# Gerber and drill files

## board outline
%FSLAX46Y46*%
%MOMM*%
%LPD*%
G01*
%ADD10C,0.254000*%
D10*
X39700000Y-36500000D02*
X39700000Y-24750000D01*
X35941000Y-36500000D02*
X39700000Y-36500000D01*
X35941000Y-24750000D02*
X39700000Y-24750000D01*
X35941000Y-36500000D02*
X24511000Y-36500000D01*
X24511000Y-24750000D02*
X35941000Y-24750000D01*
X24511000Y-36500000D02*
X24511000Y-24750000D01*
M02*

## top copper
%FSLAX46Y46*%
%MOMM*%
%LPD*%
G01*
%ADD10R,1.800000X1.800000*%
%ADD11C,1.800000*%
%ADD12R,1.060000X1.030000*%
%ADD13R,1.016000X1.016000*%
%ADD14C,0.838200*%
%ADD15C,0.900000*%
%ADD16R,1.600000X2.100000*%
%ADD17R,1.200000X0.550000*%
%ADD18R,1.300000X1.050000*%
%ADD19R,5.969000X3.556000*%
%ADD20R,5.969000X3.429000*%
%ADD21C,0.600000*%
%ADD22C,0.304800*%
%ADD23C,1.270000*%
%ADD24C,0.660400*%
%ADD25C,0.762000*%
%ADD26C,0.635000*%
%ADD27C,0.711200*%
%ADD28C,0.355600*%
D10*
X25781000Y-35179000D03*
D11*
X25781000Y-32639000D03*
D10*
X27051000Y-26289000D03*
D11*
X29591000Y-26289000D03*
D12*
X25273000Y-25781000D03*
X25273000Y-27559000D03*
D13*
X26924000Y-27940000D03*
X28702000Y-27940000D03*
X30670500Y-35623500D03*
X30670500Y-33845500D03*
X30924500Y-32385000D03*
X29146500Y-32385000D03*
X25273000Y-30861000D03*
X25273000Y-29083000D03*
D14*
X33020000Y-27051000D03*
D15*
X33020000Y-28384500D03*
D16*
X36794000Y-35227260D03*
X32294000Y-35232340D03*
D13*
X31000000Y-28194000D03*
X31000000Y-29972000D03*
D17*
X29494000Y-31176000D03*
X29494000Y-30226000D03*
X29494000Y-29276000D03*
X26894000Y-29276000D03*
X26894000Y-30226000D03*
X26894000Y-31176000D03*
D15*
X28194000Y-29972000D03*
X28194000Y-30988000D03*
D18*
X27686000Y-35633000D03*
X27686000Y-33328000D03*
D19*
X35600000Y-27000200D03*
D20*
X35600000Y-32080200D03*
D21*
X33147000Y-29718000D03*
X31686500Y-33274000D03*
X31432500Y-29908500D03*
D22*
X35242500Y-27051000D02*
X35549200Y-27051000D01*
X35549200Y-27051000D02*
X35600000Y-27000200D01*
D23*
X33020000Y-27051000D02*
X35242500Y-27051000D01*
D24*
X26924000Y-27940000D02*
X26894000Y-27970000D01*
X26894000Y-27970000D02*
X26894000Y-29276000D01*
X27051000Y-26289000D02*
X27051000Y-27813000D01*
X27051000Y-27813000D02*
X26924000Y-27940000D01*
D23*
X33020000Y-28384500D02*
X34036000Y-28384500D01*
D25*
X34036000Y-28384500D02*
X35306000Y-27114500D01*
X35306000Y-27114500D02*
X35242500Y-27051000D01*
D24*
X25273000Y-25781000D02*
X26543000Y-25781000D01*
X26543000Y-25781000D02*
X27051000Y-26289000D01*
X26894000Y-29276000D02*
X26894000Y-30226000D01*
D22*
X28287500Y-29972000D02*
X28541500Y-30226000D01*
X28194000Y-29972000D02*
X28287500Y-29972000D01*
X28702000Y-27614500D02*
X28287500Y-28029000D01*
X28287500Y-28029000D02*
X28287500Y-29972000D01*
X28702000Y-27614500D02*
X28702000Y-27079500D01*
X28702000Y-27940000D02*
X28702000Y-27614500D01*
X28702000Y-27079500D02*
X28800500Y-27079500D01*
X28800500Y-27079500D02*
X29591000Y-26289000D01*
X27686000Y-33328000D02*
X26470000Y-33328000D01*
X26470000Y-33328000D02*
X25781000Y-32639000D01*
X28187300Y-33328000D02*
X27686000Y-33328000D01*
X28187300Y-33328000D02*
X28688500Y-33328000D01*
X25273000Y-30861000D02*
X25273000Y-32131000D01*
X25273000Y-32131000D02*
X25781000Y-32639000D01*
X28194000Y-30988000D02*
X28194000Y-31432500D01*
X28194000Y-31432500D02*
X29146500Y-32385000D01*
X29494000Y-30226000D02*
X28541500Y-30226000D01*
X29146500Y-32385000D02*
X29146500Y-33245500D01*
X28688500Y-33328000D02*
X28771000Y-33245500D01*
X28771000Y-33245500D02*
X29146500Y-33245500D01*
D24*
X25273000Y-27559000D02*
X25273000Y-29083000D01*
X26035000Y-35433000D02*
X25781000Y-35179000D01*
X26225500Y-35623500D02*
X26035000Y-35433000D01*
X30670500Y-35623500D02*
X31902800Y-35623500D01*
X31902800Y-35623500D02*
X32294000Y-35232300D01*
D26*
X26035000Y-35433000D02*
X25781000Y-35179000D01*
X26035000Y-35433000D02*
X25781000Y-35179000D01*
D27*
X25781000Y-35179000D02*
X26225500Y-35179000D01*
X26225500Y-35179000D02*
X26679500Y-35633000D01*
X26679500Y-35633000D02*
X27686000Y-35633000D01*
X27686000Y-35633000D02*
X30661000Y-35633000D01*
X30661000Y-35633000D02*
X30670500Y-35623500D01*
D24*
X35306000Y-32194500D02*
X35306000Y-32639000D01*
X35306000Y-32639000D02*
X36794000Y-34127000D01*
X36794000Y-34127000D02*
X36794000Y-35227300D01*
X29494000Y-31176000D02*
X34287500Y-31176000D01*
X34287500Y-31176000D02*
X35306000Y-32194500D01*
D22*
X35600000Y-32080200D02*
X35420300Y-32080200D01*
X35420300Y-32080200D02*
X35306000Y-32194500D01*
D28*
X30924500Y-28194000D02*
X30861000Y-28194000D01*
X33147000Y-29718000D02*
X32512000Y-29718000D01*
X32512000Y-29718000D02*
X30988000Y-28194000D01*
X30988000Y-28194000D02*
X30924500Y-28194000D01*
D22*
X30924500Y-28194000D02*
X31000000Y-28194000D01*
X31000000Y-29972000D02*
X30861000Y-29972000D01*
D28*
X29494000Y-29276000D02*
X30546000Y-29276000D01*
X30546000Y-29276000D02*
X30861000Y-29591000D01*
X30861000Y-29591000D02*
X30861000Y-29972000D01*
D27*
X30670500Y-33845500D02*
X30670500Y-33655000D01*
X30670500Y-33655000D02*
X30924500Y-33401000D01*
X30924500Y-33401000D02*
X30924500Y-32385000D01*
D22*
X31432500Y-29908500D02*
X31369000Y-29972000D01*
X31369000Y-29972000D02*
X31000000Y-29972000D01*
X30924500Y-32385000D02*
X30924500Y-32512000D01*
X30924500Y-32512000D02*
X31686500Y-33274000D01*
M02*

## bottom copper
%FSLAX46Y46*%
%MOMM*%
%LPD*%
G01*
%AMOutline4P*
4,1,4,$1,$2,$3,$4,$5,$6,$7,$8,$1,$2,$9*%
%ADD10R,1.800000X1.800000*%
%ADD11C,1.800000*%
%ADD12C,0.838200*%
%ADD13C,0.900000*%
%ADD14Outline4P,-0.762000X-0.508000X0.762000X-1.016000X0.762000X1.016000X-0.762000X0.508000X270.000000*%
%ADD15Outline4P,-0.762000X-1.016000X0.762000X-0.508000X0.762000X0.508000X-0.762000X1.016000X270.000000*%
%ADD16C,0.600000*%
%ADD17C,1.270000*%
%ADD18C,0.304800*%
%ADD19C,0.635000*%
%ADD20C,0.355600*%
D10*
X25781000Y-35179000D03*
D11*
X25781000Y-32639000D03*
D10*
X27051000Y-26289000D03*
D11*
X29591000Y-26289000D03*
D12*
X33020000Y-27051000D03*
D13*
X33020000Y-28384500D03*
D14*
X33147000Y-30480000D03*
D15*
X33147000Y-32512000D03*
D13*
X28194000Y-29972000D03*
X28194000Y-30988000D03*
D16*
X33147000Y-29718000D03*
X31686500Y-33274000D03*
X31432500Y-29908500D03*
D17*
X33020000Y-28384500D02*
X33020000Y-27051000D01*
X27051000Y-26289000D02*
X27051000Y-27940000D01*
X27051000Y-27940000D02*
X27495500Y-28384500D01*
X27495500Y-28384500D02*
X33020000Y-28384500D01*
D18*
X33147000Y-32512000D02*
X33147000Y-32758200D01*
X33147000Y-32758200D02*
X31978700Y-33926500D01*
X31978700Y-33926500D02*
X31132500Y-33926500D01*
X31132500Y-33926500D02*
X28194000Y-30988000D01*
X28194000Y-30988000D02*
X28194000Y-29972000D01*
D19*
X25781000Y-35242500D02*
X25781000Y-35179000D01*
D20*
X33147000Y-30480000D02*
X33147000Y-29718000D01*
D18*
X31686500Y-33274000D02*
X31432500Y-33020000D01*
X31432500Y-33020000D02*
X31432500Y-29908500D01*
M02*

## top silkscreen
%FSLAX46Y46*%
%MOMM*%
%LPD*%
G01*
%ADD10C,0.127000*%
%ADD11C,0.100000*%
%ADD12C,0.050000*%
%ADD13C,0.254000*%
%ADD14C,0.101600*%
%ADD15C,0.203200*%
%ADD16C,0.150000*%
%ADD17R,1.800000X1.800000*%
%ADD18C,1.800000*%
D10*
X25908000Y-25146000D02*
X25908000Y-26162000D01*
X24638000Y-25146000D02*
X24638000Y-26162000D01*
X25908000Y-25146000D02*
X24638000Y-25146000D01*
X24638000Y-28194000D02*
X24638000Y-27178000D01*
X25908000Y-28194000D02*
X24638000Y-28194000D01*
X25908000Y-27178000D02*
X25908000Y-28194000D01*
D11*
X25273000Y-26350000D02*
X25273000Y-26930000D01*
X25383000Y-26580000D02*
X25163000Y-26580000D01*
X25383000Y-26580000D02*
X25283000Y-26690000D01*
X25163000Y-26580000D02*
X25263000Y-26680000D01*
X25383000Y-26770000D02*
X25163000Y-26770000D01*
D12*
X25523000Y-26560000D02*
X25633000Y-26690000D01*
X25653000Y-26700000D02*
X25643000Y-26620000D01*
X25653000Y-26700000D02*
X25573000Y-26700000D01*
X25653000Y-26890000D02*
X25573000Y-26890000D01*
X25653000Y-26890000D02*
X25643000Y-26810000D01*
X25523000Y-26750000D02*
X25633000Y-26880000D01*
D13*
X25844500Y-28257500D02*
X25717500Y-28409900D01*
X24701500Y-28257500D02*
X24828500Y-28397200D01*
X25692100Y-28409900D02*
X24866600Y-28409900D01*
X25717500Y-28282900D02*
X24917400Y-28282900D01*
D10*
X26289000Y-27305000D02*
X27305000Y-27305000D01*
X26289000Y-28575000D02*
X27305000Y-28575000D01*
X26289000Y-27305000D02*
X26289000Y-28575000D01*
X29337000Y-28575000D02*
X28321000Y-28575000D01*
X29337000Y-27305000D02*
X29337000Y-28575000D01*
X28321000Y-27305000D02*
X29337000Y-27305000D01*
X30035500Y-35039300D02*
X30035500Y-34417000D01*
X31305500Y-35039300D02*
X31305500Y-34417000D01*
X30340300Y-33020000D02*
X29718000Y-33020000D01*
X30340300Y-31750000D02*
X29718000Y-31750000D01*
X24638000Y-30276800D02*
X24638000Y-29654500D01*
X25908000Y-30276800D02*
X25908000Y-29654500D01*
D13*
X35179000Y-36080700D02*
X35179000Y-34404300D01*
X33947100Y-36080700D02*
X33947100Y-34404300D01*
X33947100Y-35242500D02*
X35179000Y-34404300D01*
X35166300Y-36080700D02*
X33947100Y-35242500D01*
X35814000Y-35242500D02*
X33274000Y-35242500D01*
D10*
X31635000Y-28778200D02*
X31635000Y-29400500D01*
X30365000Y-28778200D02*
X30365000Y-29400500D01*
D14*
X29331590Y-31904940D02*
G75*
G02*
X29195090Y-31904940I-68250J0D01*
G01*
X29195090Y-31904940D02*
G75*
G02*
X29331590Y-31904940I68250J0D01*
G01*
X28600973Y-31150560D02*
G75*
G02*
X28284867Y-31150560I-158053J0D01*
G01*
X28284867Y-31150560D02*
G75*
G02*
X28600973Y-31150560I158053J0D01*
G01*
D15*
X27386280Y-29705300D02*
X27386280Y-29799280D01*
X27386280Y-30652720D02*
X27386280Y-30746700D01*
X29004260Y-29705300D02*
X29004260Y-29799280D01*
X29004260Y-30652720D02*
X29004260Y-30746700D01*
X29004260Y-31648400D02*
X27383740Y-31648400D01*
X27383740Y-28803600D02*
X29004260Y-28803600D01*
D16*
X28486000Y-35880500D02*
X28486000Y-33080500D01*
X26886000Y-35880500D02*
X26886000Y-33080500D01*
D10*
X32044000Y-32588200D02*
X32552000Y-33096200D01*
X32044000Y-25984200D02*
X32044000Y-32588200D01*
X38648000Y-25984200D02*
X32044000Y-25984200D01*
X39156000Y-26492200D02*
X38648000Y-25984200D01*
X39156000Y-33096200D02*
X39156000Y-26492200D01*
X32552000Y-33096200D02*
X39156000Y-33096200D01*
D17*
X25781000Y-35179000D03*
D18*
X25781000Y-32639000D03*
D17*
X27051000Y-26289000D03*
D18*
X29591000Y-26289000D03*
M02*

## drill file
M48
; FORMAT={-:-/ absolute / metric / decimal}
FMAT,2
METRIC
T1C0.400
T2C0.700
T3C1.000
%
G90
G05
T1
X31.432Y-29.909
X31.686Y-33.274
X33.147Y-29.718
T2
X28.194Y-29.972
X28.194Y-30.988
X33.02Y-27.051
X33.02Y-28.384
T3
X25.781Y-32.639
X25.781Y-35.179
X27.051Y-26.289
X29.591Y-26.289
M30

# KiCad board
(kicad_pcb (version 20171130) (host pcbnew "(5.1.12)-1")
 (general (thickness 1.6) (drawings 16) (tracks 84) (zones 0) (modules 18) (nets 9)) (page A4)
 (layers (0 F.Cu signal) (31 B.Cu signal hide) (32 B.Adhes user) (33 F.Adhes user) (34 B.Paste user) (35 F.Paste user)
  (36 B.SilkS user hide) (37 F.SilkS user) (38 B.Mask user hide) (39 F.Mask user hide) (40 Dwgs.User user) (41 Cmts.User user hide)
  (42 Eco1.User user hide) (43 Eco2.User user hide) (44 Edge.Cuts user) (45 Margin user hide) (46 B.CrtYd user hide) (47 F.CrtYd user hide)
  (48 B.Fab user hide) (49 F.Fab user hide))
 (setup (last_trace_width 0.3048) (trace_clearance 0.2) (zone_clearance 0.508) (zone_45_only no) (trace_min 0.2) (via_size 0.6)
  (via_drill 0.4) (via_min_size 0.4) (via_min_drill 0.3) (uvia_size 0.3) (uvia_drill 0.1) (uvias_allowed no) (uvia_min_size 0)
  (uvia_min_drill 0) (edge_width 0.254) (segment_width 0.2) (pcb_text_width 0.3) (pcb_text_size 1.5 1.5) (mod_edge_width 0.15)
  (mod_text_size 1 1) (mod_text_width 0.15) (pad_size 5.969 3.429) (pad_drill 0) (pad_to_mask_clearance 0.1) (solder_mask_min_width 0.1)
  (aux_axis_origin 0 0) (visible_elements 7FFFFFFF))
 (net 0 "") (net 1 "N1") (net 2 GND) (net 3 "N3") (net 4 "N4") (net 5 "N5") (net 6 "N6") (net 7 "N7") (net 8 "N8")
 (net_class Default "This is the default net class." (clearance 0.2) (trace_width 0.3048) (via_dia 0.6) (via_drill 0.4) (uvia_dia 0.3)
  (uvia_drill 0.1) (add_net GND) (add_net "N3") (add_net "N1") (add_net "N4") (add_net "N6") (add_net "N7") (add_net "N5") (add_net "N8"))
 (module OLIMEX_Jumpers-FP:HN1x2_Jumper (layer F.Cu) (at 25.781 33.909 90)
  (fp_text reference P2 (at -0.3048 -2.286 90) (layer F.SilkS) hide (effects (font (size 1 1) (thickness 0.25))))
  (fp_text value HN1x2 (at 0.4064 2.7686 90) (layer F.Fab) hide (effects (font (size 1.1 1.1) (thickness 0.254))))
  (pad 1 thru_hole rect (at -1.27 0 180) (size 1.8 1.8) (drill 1) (layers *.Cu *.Mask F.SilkS) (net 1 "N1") (solder_mask_margin 0.0508)
   (solder_paste_margin -0.0508))
  (pad 2 thru_hole circle (at 1.27 0 180) (size 1.8 1.8) (drill 1) (layers *.Cu *.Mask F.SilkS) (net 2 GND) (solder_mask_margin 0.0508)
   (solder_paste_margin -0.0508)))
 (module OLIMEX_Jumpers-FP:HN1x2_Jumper (layer F.Cu) (at 28.321 26.289)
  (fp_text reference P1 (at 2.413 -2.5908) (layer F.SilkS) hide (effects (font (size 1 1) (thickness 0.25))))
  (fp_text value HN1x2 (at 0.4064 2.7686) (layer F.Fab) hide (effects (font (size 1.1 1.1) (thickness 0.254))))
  (pad 1 thru_hole rect (at -1.27 0 90) (size 1.8 1.8) (drill 1) (layers *.Cu *.Mask F.SilkS) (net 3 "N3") (solder_mask_margin 0.0508)
   (solder_paste_margin -0.0508))
  (pad 2 thru_hole circle (at 1.27 0 90) (size 1.8 1.8) (drill 1) (layers *.Cu *.Mask F.SilkS) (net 2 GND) (solder_mask_margin 0.0508)
   (solder_paste_margin -0.0508)))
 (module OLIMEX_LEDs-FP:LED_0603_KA (layer F.Cu) (at 25.273 26.67 270)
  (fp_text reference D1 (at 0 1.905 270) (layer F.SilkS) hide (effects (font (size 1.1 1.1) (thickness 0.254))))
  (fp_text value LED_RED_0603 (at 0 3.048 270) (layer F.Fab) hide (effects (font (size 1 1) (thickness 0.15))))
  (fp_line (start -1.524 -0.635) (end -0.508 -0.635) (layer F.SilkS) (width 0.127))
  (fp_line (start -1.524 0.635) (end -0.508 0.635) (layer F.SilkS) (width 0.127))
  (fp_line (start -1.524 -0.635) (end -1.524 0.635) (layer F.SilkS) (width 0.127))
  (fp_line (start 1.524 0.635) (end 0.508 0.635) (layer F.SilkS) (width 0.127))
  (fp_line (start 1.524 -0.635) (end 1.524 0.635) (layer F.SilkS) (width 0.127))
  (fp_line (start 0.508 -0.635) (end 1.524 -0.635) (layer F.SilkS) (width 0.127))
  (fp_line (start -0.32 0) (end 0.26 0) (layer F.SilkS) (width 0.1))
  (fp_line (start -0.09 -0.11) (end -0.09 0.11) (layer F.SilkS) (width 0.1))
  (fp_line (start -0.09 -0.11) (end 0.02 -0.01) (layer F.SilkS) (width 0.1))
  (fp_line (start -0.09 0.11) (end 0.01 0.01) (layer F.SilkS) (width 0.1))
  (fp_line (start 0.1 -0.11) (end 0.1 0.11) (layer F.SilkS) (width 0.1))
  (fp_line (start -0.11 -0.25) (end 0.02 -0.36) (layer F.SilkS) (width 0.05))
  (fp_line (start 0.03 -0.38) (end -0.05 -0.37) (layer F.SilkS) (width 0.05))
  (fp_line (start 0.03 -0.38) (end 0.03 -0.3) (layer F.SilkS) (width 0.05))
  (fp_line (start 0.22 -0.38) (end 0.22 -0.3) (layer F.SilkS) (width 0.05))
  (fp_line (start 0.22 -0.38) (end 0.14 -0.37) (layer F.SilkS) (width 0.05))
  (fp_line (start 0.08 -0.25) (end 0.21 -0.36) (layer F.SilkS) (width 0.05))
  (fp_line (start 1.5875 -0.5715) (end 1.7399 -0.4445) (layer F.SilkS) (width 0.254))
  (fp_line (start 1.5875 0.5715) (end 1.7272 0.4445) (layer F.SilkS) (width 0.254))
  (fp_line (start 1.7399 -0.4191) (end 1.7399 0.4064) (layer F.SilkS) (width 0.254))
  (fp_line (start 1.6129 -0.4445) (end 1.6129 0.3556) (layer F.SilkS) (width 0.254))
  (pad 2 smd rect (at -0.889 0 270) (size 1.03 1.06) (layers F.Cu F.Paste F.Mask) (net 3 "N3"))
  (pad 1 smd rect (at 0.889 0 270) (size 1.03 1.06) (layers F.Cu F.Paste F.Mask) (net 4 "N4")))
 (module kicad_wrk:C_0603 (layer F.Cu) (at 27.813 27.94)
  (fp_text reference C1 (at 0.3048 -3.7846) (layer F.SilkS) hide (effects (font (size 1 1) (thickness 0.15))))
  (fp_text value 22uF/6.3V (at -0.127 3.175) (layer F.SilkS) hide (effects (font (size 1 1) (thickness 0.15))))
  (fp_line (start -1.524 -0.635) (end -0.508 -0.635) (layer F.SilkS) (width 0.127))
  (fp_line (start -1.524 0.635) (end -0.508 0.635) (layer F.SilkS) (width 0.127))
  (fp_line (start -1.524 -0.635) (end -1.524 0.635) (layer F.SilkS) (width 0.127))
  (fp_line (start 1.524 0.635) (end 0.508 0.635) (layer F.SilkS) (width 0.127))
  (fp_line (start 1.524 -0.635) (end 1.524 0.635) (layer F.SilkS) (width 0.127))
  (fp_line (start 0.508 -0.635) (end 1.524 -0.635) (layer F.SilkS) (width 0.127))
  (pad 1 smd rect (at -0.889 0) (size 1.016 1.016) (layers F.Cu F.Paste F.Mask) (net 3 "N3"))
  (pad 2 smd rect (at 0.889 0) (size 1.016 1.016) (layers F.Cu F.Paste F.Mask) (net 2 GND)))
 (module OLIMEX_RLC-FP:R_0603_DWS (layer F.Cu) (at 30.6705 34.7345 90)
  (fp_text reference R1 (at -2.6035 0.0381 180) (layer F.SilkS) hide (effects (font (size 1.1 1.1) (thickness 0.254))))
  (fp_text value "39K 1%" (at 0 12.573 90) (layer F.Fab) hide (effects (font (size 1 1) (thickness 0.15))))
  (fp_line (start -0.3048 -0.635) (end 0.3175 -0.635) (layer F.SilkS) (width 0.127))
  (fp_line (start -0.3048 0.635) (end 0.3175 0.635) (layer F.SilkS) (width 0.127))
  (pad 1 smd rect (at -0.889 0 90) (size 1.016 1.016) (layers F.Cu F.Paste F.Mask) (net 1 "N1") (solder_mask_margin 0.0508)
   (solder_paste_margin -0.0508) (clearance 0.0508))
  (pad 2 smd rect (at 0.889 0 90) (size 1.016 1.016) (layers F.Cu F.Paste F.Mask) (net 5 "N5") (solder_mask_margin 0.0508)
   (solder_paste_margin -0.0508) (clearance 0.0508)))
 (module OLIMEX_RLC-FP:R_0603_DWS (layer F.Cu) (at 30.0355 32.385 180)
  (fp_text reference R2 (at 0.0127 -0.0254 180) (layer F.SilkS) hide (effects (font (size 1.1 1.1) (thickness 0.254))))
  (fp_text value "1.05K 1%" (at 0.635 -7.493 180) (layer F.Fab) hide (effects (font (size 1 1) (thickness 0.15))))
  (fp_line (start -0.3048 -0.635) (end 0.3175 -0.635) (layer F.SilkS) (width 0.127))
  (fp_line (start -0.3048 0.635) (end 0.3175 0.635) (layer F.SilkS) (width 0.127))
  (pad 1 smd rect (at -0.889 0 180) (size 1.016 1.016) (layers F.Cu F.Paste F.Mask) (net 5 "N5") (solder_mask_margin 0.0508)
   (solder_paste_margin -0.0508) (clearance 0.0508))
  (pad 2 smd rect (at 0.889 0 180) (size 1.016 1.016) (layers F.Cu F.Paste F.Mask) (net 2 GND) (solder_mask_margin 0.0508)
   (solder_paste_margin -0.0508) (clearance 0.0508)))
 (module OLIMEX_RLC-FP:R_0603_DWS (layer F.Cu) (at 25.273 29.972 90)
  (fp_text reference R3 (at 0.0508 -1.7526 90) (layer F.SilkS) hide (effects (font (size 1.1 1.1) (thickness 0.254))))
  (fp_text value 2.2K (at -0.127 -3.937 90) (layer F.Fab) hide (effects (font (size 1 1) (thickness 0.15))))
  (fp_line (start -0.3048 -0.635) (end 0.3175 -0.635) (layer F.SilkS) (width 0.127))
  (fp_line (start -0.3048 0.635) (end 0.3175 0.635) (layer F.SilkS) (width 0.127))
  (pad 1 smd rect (at -0.889 0 90) (size 1.016 1.016) (layers F.Cu F.Paste F.Mask) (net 2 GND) (solder_mask_margin 0.0508)
   (solder_paste_margin -0.0508) (clearance 0.0508))
  (pad 2 smd rect (at 0.889 0 90) (size 1.016 1.016) (layers F.Cu F.Paste F.Mask) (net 4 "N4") (solder_mask_margin 0.0508)
   (solder_paste_margin -0.0508) (clearance 0.0508)))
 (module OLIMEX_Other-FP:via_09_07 (layer F.Cu) (at 33.02 27.051 180)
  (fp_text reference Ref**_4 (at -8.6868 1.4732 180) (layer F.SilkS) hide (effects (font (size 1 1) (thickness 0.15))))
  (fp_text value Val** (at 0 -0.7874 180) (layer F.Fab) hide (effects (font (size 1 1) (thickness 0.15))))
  (pad 0 thru_hole circle (at 0 0 180) (size 0.8382 0.8382) (drill 0.7) (layers *.Cu) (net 3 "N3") (zone_connect 2)))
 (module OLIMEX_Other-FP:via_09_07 (layer F.Cu) (at 33.02 28.321 180)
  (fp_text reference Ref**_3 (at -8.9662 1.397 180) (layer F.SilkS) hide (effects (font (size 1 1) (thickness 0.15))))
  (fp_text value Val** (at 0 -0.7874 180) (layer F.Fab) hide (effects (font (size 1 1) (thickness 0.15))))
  (pad 0 thru_hole circle (at 0 -0.0635 180) (size 0.9 0.9) (drill 0.7) (layers *.Cu) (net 3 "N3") (zone_connect 2)))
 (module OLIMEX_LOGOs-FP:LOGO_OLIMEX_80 (layer B.Cu) (at 35.8775 27.686 180)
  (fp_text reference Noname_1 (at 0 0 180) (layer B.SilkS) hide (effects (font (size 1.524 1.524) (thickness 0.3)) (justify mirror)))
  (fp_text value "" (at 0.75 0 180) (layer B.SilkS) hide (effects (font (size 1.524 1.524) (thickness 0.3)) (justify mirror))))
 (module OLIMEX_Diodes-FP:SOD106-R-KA (layer F.Cu) (at 34.544 35.2425 180)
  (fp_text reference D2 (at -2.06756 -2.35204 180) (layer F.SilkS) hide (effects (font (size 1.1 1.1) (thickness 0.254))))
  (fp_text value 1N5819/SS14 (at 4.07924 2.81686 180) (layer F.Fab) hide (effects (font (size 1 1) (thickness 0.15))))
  (fp_line (start -0.635 -0.8382) (end -0.635 0.8382) (layer F.SilkS) (width 0.254))
  (fp_line (start 0.5969 -0.8382) (end 0.5969 0.8382) (layer F.SilkS) (width 0.254))
  (fp_line (start 0.5969 0) (end -0.635 0.8382) (layer F.SilkS) (width 0.254))
  (fp_line (start -0.6223 -0.8382) (end 0.5969 0) (layer F.SilkS) (width 0.254))
  (fp_line (start -1.27 0) (end 1.27 0) (layer F.SilkS) (width 0.254))
  (pad 2 smd rect (at -2.25 0.01524 180) (size 1.6 2.1) (layers F.Cu F.Paste F.Mask) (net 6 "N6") (solder_mask_margin 0.0508)
   (solder_paste_margin -0.0508) (clearance 0.0508))
  (pad 1 smd rect (at 2.25 0.01016 180) (size 1.6 2.1) (layers F.Cu F.Paste F.Mask) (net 1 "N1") (solder_mask_margin 0.0508)
   (solder_paste_margin -0.0508) (clearance 0.0508)))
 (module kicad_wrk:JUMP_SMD (layer B.Cu) (at 33.147 31.496 270)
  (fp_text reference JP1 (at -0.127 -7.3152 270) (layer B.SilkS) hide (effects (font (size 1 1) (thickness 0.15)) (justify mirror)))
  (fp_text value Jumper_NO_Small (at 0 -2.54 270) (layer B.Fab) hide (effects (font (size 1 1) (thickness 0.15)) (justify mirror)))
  (pad 1 smd trapezoid (at -1.016 0 270) (size 1.524 1.524) (rect_delta -0.508 0) (layers B.Cu B.Mask) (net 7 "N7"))
  (pad 2 smd trapezoid (at 1.016 0 270) (size 1.524 1.524) (rect_delta 0.508 0) (layers B.Cu B.Mask) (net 2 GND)))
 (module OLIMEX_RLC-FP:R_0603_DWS (layer F.Cu) (at 31 29.083 270)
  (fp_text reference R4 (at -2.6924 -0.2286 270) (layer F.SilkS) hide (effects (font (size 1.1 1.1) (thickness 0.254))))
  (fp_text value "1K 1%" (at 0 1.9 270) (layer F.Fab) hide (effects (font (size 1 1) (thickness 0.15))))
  (fp_line (start -0.3048 -0.635) (end 0.3175 -0.635) (layer F.SilkS) (width 0.127))
  (fp_line (start -0.3048 0.635) (end 0.3175 0.635) (layer F.SilkS) (width 0.127))
  (pad 1 smd rect (at -0.889 0 270) (size 1.016 1.016) (layers F.Cu F.Paste F.Mask) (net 7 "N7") (solder_mask_margin 0.0508)
   (solder_paste_margin -0.0508) (clearance 0.0508))
  (pad 2 smd rect (at 0.889 0 270) (size 1.016 1.016) (layers F.Cu F.Paste F.Mask) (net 5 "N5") (solder_mask_margin 0.0508)
   (solder_paste_margin -0.0508) (clearance 0.0508)))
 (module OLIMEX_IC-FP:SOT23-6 (layer F.Cu) (at 28.194 30.226)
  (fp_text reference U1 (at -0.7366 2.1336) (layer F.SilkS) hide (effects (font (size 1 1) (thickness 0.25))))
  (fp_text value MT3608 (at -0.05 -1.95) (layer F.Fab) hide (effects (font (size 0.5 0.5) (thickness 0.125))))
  (fp_circle (center 1.06934 1.67894) (end 1.1176 1.7272) (layer F.SilkS) (width 0.1016))
  (fp_circle (center 0.24892 0.92456) (end 0.36068 1.03632) (layer F.SilkS) (width 0.1016))
  (fp_line (start -0.80772 -0.5207) (end -0.80772 -0.42672) (layer F.SilkS) (width 0.2032))
  (fp_line (start -0.80772 0.42672) (end -0.80772 0.5207) (layer F.SilkS) (width 0.2032))
  (fp_line (start 0.81026 -0.5207) (end 0.81026 -0.42672) (layer F.SilkS) (width 0.2032))
  (fp_line (start 0.81026 0.42672) (end 0.81026 0.5207) (layer F.SilkS) (width 0.2032))
  (fp_line (start 0.81026 1.4224) (end -0.81026 1.4224) (layer F.SilkS) (width 0.2032))
  (fp_line (start -0.81026 -1.4224) (end 0.81026 -1.4224) (layer F.SilkS) (width 0.2032))
  (pad 1 smd rect (at 1.3 0.95 90) (size 0.55 1.2) (layers F.Cu F.Paste F.Mask) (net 6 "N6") (solder_mask_margin 0.0508)
   (solder_paste_margin -0.0508) (clearance 0.0508))
  (pad 2 smd rect (at 1.3 0 90) (size 0.55 1.2) (layers F.Cu F.Paste F.Mask) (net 2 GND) (solder_mask_margin 0.0508)
   (solder_paste_margin -0.0508) (clearance 0.0508))
  (pad 3 smd rect (at 1.3 -0.95 90) (size 0.55 1.2) (layers F.Cu F.Paste F.Mask) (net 5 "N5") (solder_mask_margin 0.0508)
   (solder_paste_margin -0.0508) (clearance 0.0508))
  (pad 4 smd rect (at -1.3 -0.95 90) (size 0.55 1.2) (layers F.Cu F.Paste F.Mask) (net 3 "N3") (solder_mask_margin 0.0508)
   (solder_paste_margin -0.0508) (clearance 0.0508))
  (pad 5 smd rect (at -1.3 0 90) (size 0.55 1.2) (layers F.Cu F.Paste F.Mask) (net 3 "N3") (solder_mask_margin 0.0508)
   (solder_paste_margin -0.0508) (clearance 0.0508))
  (pad 6 smd rect (at -1.3 0.95 90) (size 0.55 1.2) (layers F.Cu F.Paste F.Mask) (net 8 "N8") (solder_mask_margin 0.0508)
   (solder_paste_margin -0.0508) (clearance 0.0508)))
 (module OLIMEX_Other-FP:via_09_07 (layer F.Cu) (at 28.194 29.972)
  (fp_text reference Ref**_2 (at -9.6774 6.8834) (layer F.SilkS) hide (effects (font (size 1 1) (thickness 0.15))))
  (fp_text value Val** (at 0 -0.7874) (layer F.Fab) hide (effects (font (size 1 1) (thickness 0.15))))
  (pad 0 thru_hole circle (at 0 0) (size 0.9 0.9) (drill 0.7) (layers *.Cu) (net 2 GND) (zone_connect 2)))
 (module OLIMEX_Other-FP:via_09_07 (layer F.Cu) (at 28.194 30.988)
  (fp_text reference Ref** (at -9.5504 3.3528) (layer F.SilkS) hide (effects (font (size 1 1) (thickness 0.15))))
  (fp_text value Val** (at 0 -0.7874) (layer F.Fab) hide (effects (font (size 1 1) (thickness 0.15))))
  (pad 0 thru_hole circle (at 0 0) (size 0.9 0.9) (drill 0.7) (layers *.Cu) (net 2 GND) (zone_connect 2)))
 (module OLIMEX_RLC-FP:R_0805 (layer F.Cu) (at 27.686 34.4805 180)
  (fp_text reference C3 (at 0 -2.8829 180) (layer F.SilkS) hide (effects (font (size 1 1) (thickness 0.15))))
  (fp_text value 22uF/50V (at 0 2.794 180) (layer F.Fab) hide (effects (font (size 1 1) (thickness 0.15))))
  (fp_line (start -0.8 -1.4) (end -0.8 1.4) (layer F.SilkS) (width 0.15))
  (fp_line (start 0.8 -1.4) (end 0.8 1.4) (layer F.SilkS) (width 0.15))
  (pad 1 smd rect (at 0 -1.1525 180) (size 1.3 1.05) (layers F.Cu F.Paste F.Mask) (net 1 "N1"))
  (pad 2 smd rect (at 0 1.1525 180) (size 1.3 1.05) (layers F.Cu F.Paste F.Mask) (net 2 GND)))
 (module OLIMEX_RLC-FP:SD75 (layer F.Cu) (at 35.6 29.5402)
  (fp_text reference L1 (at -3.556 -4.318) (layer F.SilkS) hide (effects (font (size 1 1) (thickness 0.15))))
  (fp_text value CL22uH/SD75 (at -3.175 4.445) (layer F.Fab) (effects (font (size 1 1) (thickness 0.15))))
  (fp_line (start -3.556 3.048) (end -3.048 3.556) (layer F.SilkS) (width 0.127))
  (fp_line (start -3.556 -3.556) (end -3.556 3.048) (layer F.SilkS) (width 0.127))
  (fp_line (start 3.048 -3.556) (end -3.556 -3.556) (layer F.SilkS) (width 0.127))
  (fp_line (start 3.556 -3.048) (end 3.048 -3.556) (layer F.SilkS) (width 0.127))
  (fp_line (start 3.556 3.556) (end 3.556 -3.048) (layer F.SilkS) (width 0.127))
  (fp_line (start -3.048 3.556) (end 3.556 3.556) (layer F.SilkS) (width 0.127))
  (pad 1 smd rect (at 0 -2.54) (size 5.969 3.556) (layers F.Cu F.Paste F.Mask) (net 3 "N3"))
  (pad 2 smd rect (at 0 2.54) (size 5.969 3.429) (layers F.Cu F.Paste F.Mask) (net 6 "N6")))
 (gr_line (start 39.7 36.5) (end 39.7 24.75) (angle 90) (layer Edge.Cuts) (width 0.254))
 (gr_line (start 35.941 36.5) (end 39.7 36.5) (angle 90) (layer Edge.Cuts) (width 0.254))
 (gr_line (start 35.941 24.75) (end 39.7 24.75) (angle 90) (layer Edge.Cuts) (width 0.254))
 (gr_line (start 35.941 36.5) (end 24.511 36.5) (angle 90) (layer Edge.Cuts) (width 0.254))
 (gr_line (start 24.511 24.75) (end 35.941 24.75) (angle 90) (layer Edge.Cuts) (width 0.254))
 (gr_line (start 24.511 36.5) (end 24.511 24.75) (angle 90) (layer Edge.Cuts) (width 0.254))
 (segment (start 35.2425 27.051) (end 35.5492 27.051) (width 0.3048) (layer F.Cu) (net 3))
 (segment (start 35.5492 27.051) (end 35.6 27.0002) (width 0.3048) (layer F.Cu) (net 3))
 (segment (start 33.02 27.051) (end 35.2425 27.051) (width 1.27) (layer F.Cu) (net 3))
 (segment (start 26.924 27.94) (end 26.894 27.97) (width 0.6604) (layer F.Cu) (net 3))
 (segment (start 26.894 27.97) (end 26.894 29.276) (width 0.6604) (layer F.Cu) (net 3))
 (segment (start 27.051 26.289) (end 27.051 27.813) (width 0.6604) (layer F.Cu) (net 3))
 (segment (start 27.051 27.813) (end 26.924 27.94) (width 0.6604) (layer F.Cu) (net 3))
 (segment (start 33.02 28.3845) (end 33.02 27.051) (width 1.27) (layer B.Cu) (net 3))
 (segment (start 27.051 26.289) (end 27.051 27.94) (width 1.27) (layer B.Cu) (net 3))
 (segment (start 27.051 27.94) (end 27.4955 28.3845) (width 1.27) (layer B.Cu) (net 3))
 (segment (start 27.4955 28.3845) (end 33.02 28.3845) (width 1.27) (layer B.Cu) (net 3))
 (segment (start 33.02 28.3845) (end 34.036 28.3845) (width 1.27) (layer F.Cu) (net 3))
 (segment (start 34.036 28.3845) (end 35.306 27.1145) (width 0.762) (layer F.Cu) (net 3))
 (segment (start 35.306 27.1145) (end 35.2425 27.051) (width 0.762) (layer F.Cu) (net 3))
 (segment (start 25.273 25.781) (end 26.543 25.781) (width 0.6604) (layer F.Cu) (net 3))
 (segment (start 26.543 25.781) (end 27.051 26.289) (width 0.6604) (layer F.Cu) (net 3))
 (segment (start 26.894 29.276) (end 26.894 30.226) (width 0.6604) (layer F.Cu) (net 3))
 (segment (start 28.2875 29.972) (end 28.5415 30.226) (width 0.3048) (layer F.Cu) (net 2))
 (segment (start 28.194 29.972) (end 28.2875 29.972) (width 0.3048) (layer F.Cu) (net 2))
 (segment (start 28.702 27.6145) (end 28.2875 28.029) (width 0.3048) (layer F.Cu) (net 2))
 (segment (start 28.2875 28.029) (end 28.2875 29.972) (width 0.3048) (layer F.Cu) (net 2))
 (segment (start 28.702 27.6145) (end 28.702 27.0795) (width 0.3048) (layer F.Cu) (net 2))
 (segment (start 28.702 27.94) (end 28.702 27.6145) (width 0.3048) (layer F.Cu) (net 2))
 (segment (start 28.702 27.0795) (end 28.8005 27.0795) (width 0.3048) (layer F.Cu) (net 2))
 (segment (start 28.8005 27.0795) (end 29.591 26.289) (width 0.3048) (layer F.Cu) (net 2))
 (segment (start 27.686 33.328) (end 26.47 33.328) (width 0.3048) (layer F.Cu) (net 2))
 (segment (start 26.47 33.328) (end 25.781 32.639) (width 0.3048) (layer F.Cu) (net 2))
 (segment (start 28.1873 33.328) (end 27.686 33.328) (width 0.3048) (layer F.Cu) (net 2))
 (segment (start 28.1873 33.328) (end 28.6885 33.328) (width 0.3048) (layer F.Cu) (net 2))
 (segment (start 25.273 30.861) (end 25.273 32.131) (width 0.3048) (layer F.Cu) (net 2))
 (segment (start 25.273 32.131) (end 25.781 32.639) (width 0.3048) (layer F.Cu) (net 2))
 (segment (start 33.147 32.512) (end 33.147 32.7582) (width 0.3048) (layer B.Cu) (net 2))
 (segment (start 33.147 32.7582) (end 31.9787 33.9265) (width 0.3048) (layer B.Cu) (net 2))
 (segment (start 31.9787 33.9265) (end 31.1325 33.9265) (width 0.3048) (layer B.Cu) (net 2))
 (segment (start 31.1325 33.9265) (end 28.194 30.988) (width 0.3048) (layer B.Cu) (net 2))
 (segment (start 28.194 30.988) (end 28.194 31.4325) (width 0.3048) (layer F.Cu) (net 2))
 (segment (start 28.194 31.4325) (end 29.1465 32.385) (width 0.3048) (layer F.Cu) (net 2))
 (segment (start 29.494 30.226) (end 28.5415 30.226) (width 0.3048) (layer F.Cu) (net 2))
 (segment (start 28.194 30.988) (end 28.194 29.972) (width 0.3048) (layer B.Cu) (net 2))
 (segment (start 29.1465 32.385) (end 29.1465 33.2455) (width 0.3048) (layer F.Cu) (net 2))
 (segment (start 28.6885 33.328) (end 28.771 33.2455) (width 0.3048) (layer F.Cu) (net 2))
 (segment (start 28.771 33.2455) (end 29.1465 33.2455) (width 0.3048) (layer F.Cu) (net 2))
 (segment (start 25.273 27.559) (end 25.273 29.083) (width 0.6604) (layer F.Cu) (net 4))
 (segment (start 26.035 35.433) (end 25.781 35.179) (width 0.6604) (layer F.Cu) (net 1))
 (segment (start 26.2255 35.6235) (end 26.035 35.433) (width 0.6604) (layer F.Cu) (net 1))
 (segment (start 30.6705 35.6235) (end 31.9028 35.6235) (width 0.6604) (layer F.Cu) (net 1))
 (segment (start 31.9028 35.6235) (end 32.294 35.2323) (width 0.6604) (layer F.Cu) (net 1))
 (segment (start 26.035 35.433) (end 25.781 35.179) (width 0.635) (layer F.Cu) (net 1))
 (segment (start 26.035 35.433) (end 25.781 35.179) (width 0.635) (layer F.Cu) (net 1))
 (segment (start 25.781 35.2425) (end 25.781 35.179) (width 0.635) (layer B.Cu) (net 1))
 (segment (start 25.781 35.179) (end 26.2255 35.179) (width 0.7112) (layer F.Cu) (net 1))
 (segment (start 26.2255 35.179) (end 26.6795 35.633) (width 0.7112) (layer F.Cu) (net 1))
 (segment (start 26.6795 35.633) (end 27.686 35.633) (width 0.7112) (layer F.Cu) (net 1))
 (segment (start 27.686 35.633) (end 30.661 35.633) (width 0.7112) (layer F.Cu) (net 1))
 (segment (start 30.661 35.633) (end 30.6705 35.6235) (width 0.7112) (layer F.Cu) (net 1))
 (segment (start 35.306 32.1945) (end 35.306 32.639) (width 0.6604) (layer F.Cu) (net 6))
 (segment (start 35.306 32.639) (end 36.794 34.127) (width 0.6604) (layer F.Cu) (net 6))
 (segment (start 36.794 34.127) (end 36.794 35.2273) (width 0.6604) (layer F.Cu) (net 6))
 (segment (start 29.494 31.176) (end 34.2875 31.176) (width 0.6604) (layer F.Cu) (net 6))
 (segment (start 34.2875 31.176) (end 35.306 32.1945) (width 0.6604) (layer F.Cu) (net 6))
 (segment (start 35.6 32.0802) (end 35.4203 32.0802) (width 0.3048) (layer F.Cu) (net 6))
 (segment (start 35.4203 32.0802) (end 35.306 32.1945) (width 0.3048) (layer F.Cu) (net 6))
 (segment (start 30.9245 28.194) (end 30.861 28.194) (width 0.3556) (layer F.Cu) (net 7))
 (segment (start 33.147 29.718) (end 32.512 29.718) (width 0.3556) (layer F.Cu) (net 7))
 (segment (start 32.512 29.718) (end 30.988 28.194) (width 0.3556) (layer F.Cu) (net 7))
 (segment (start 30.988 28.194) (end 30.9245 28.194) (width 0.3556) (layer F.Cu) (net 7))
 (segment (start 30.9245 28.194) (end 31 28.194) (width 0.3048) (layer F.Cu) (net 7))
 (segment (start 33.147 30.48) (end 33.147 29.718) (width 0.3556) (layer B.Cu) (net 7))
 (via (at 33.147 29.718) (size 0.6) (layers F.Cu B.Cu) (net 7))
 (segment (start 31 29.972) (end 30.861 29.972) (width 0.3048) (layer F.Cu) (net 5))
 (segment (start 29.494 29.276) (end 30.546 29.276) (width 0.3556) (layer F.Cu) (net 5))
 (segment (start 30.546 29.276) (end 30.861 29.591) (width 0.3556) (layer F.Cu) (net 5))
 (segment (start 30.861 29.591) (end 30.861 29.972) (width 0.3556) (layer F.Cu) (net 5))
 (segment (start 30.6705 33.8455) (end 30.6705 33.655) (width 0.7112) (layer F.Cu) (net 5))
 (segment (start 30.6705 33.655) (end 30.9245 33.401) (width 0.7112) (layer F.Cu) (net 5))
 (segment (start 30.9245 33.401) (end 30.9245 32.385) (width 0.7112) (layer F.Cu) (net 5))
 (segment (start 31.6865 33.274) (end 31.4325 33.02) (width 0.3048) (layer B.Cu) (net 5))
 (segment (start 31.4325 33.02) (end 31.4325 29.9085) (width 0.3048) (layer B.Cu) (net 5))
 (segment (start 31.4325 29.9085) (end 31.369 29.972) (width 0.3048) (layer F.Cu) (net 5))
 (segment (start 31.369 29.972) (end 31 29.972) (width 0.3048) (layer F.Cu) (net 5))
 (segment (start 30.9245 32.385) (end 30.9245 32.512) (width 0.3048) (layer F.Cu) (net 5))
 (segment (start 30.9245 32.512) (end 31.6865 33.274) (width 0.3048) (layer F.Cu) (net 5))
 (via (at 31.6865 33.274) (size 0.6) (layers F.Cu B.Cu) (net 5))
 (via (at 31.4325 29.9085) (size 0.6) (layers F.Cu B.Cu) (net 5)))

